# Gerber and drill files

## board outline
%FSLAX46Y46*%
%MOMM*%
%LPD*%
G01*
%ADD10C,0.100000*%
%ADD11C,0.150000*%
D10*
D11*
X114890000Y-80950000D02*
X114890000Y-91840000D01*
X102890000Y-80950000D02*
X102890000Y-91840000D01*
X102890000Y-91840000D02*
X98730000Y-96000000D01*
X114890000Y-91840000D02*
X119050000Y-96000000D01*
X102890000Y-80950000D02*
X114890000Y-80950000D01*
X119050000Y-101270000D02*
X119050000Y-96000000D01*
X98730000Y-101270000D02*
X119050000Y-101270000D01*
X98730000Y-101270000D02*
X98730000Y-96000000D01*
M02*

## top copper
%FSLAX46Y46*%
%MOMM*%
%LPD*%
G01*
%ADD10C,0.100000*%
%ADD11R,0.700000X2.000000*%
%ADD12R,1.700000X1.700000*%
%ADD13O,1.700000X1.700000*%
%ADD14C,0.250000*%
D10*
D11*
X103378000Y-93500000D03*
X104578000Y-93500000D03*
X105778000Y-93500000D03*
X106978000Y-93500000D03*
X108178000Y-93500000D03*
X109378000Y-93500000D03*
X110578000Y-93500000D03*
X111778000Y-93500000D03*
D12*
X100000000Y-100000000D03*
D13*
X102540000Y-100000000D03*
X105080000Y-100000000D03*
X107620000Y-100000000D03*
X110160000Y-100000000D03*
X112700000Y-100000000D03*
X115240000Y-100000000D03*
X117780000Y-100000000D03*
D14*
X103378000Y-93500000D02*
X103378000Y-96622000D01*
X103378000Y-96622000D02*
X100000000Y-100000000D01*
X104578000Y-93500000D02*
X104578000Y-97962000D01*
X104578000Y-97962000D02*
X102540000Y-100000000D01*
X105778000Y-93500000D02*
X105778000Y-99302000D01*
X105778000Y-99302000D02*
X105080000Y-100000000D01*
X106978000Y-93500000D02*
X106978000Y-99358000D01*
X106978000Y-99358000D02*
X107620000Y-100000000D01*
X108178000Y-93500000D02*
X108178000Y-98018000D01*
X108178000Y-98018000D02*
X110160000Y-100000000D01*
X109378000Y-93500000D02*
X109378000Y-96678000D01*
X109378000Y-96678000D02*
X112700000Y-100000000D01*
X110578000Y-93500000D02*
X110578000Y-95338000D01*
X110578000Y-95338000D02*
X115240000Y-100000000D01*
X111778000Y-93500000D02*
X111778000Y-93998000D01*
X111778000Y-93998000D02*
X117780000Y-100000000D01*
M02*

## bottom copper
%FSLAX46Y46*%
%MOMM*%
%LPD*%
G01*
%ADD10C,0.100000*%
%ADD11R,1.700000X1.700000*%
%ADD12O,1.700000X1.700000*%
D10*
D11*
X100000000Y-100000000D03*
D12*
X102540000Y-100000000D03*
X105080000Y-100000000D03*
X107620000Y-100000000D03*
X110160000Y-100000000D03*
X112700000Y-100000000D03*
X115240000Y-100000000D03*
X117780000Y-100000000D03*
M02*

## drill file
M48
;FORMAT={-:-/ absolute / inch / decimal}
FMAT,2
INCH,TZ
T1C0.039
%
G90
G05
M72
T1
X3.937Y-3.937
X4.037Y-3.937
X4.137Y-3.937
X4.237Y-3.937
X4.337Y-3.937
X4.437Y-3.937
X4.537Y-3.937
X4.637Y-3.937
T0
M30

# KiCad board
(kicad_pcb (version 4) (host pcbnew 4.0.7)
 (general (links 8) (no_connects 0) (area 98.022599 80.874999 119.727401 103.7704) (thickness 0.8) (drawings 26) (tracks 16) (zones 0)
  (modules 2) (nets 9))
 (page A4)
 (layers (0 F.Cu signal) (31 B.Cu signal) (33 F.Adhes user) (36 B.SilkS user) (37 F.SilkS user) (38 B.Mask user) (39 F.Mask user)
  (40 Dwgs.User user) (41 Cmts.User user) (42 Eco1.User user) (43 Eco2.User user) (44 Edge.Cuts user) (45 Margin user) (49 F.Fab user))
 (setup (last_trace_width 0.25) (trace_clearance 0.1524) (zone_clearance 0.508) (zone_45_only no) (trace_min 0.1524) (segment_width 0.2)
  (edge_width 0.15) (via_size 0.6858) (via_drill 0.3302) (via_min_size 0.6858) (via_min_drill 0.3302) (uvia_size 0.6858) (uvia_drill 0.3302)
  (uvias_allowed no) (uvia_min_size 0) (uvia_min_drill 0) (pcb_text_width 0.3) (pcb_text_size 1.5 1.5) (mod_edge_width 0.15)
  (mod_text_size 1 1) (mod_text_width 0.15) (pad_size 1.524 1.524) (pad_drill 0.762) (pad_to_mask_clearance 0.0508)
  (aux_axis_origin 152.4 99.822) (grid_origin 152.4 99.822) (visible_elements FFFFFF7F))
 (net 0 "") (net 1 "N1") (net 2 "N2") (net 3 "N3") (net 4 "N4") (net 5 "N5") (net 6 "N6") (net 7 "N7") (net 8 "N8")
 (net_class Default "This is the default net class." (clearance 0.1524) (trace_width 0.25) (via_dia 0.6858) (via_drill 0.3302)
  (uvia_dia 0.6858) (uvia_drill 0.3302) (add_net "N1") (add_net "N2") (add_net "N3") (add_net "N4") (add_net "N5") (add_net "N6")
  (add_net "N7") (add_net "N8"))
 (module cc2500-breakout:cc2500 (layer F.Cu) (at 103.378 93.5)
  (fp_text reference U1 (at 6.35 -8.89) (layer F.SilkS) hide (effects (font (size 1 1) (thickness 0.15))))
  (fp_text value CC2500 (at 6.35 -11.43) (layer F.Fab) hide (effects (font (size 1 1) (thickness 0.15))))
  (pad 1 smd rect (at 0 0) (size 0.7 2) (layers F.Cu F.Mask) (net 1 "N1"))
  (pad 2 smd rect (at 1.2 0) (size 0.7 2) (layers F.Cu F.Mask) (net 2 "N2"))
  (pad 3 smd rect (at 2.4 0) (size 0.7 2) (layers F.Cu F.Mask) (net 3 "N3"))
  (pad 4 smd rect (at 3.6 0) (size 0.7 2) (layers F.Cu F.Mask) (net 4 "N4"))
  (pad 5 smd rect (at 4.8 0) (size 0.7 2) (layers F.Cu F.Mask) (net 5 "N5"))
  (pad 6 smd rect (at 6 0) (size 0.7 2) (layers F.Cu F.Mask) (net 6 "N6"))
  (pad 7 smd rect (at 7.2 0) (size 0.7 2) (layers F.Cu F.Mask) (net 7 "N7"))
  (pad 8 smd rect (at 8.4 0) (size 0.7 2) (layers F.Cu F.Mask) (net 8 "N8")))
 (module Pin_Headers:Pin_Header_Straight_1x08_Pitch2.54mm (layer F.Cu) (at 100 100 90)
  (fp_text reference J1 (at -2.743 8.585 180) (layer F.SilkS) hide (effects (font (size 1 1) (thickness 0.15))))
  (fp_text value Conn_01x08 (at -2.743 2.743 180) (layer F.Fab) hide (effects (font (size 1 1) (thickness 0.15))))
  (pad 1 thru_hole rect (at 0 0 90) (size 1.7 1.7) (drill 1) (layers *.Cu *.Mask) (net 1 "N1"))
  (pad 2 thru_hole oval (at 0 2.54 90) (size 1.7 1.7) (drill 1) (layers *.Cu *.Mask) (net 2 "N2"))
  (pad 3 thru_hole oval (at 0 5.08 90) (size 1.7 1.7) (drill 1) (layers *.Cu *.Mask) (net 3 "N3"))
  (pad 4 thru_hole oval (at 0 7.62 90) (size 1.7 1.7) (drill 1) (layers *.Cu *.Mask) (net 4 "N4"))
  (pad 5 thru_hole oval (at 0 10.16 90) (size 1.7 1.7) (drill 1) (layers *.Cu *.Mask) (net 5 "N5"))
  (pad 6 thru_hole oval (at 0 12.7 90) (size 1.7 1.7) (drill 1) (layers *.Cu *.Mask) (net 6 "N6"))
  (pad 7 thru_hole oval (at 0 15.24 90) (size 1.7 1.7) (drill 1) (layers *.Cu *.Mask) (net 7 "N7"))
  (pad 8 thru_hole oval (at 0 17.78 90) (size 1.7 1.7) (drill 1) (layers *.Cu *.Mask) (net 8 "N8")))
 (gr_line (start 114.89 80.95) (end 114.89 91.84) (angle 90) (layer Edge.Cuts) (width 0.15))
 (gr_line (start 102.89 80.95) (end 102.89 91.84) (angle 90) (layer Edge.Cuts) (width 0.15))
 (gr_line (start 102.89 91.84) (end 98.73 96) (angle 90) (layer Edge.Cuts) (width 0.15))
 (gr_line (start 114.89 91.84) (end 119.05 96) (angle 90) (layer Edge.Cuts) (width 0.15))
 (gr_line (start 102.89 80.95) (end 114.89 80.95) (angle 90) (layer Edge.Cuts) (width 0.15))
 (gr_line (start 119.05 101.27) (end 119.05 96) (angle 90) (layer Edge.Cuts) (width 0.15))
 (gr_line (start 98.73 101.27) (end 119.05 101.27) (angle 90) (layer Edge.Cuts) (width 0.15))
 (gr_line (start 98.73 101.27) (end 98.73 96) (angle 90) (layer Edge.Cuts) (width 0.15))
 (segment (start 103.378 93.5) (end 103.378 96.622) (width 0.25) (layer F.Cu) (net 1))
 (segment (start 103.378 96.622) (end 100 100) (width 0.25) (layer F.Cu) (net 1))
 (segment (start 104.578 93.5) (end 104.578 97.962) (width 0.25) (layer F.Cu) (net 2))
 (segment (start 104.578 97.962) (end 102.54 100) (width 0.25) (layer F.Cu) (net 2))
 (segment (start 105.778 93.5) (end 105.778 99.302) (width 0.25) (layer F.Cu) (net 3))
 (segment (start 105.778 99.302) (end 105.08 100) (width 0.25) (layer F.Cu) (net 3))
 (segment (start 106.978 93.5) (end 106.978 99.358) (width 0.25) (layer F.Cu) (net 4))
 (segment (start 106.978 99.358) (end 107.62 100) (width 0.25) (layer F.Cu) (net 4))
 (segment (start 108.178 93.5) (end 108.178 98.018) (width 0.25) (layer F.Cu) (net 5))
 (segment (start 108.178 98.018) (end 110.16 100) (width 0.25) (layer F.Cu) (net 5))
 (segment (start 109.378 93.5) (end 109.378 96.678) (width 0.25) (layer F.Cu) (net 6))
 (segment (start 109.378 96.678) (end 112.7 100) (width 0.25) (layer F.Cu) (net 6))
 (segment (start 110.578 93.5) (end 110.578 95.338) (width 0.25) (layer F.Cu) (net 7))
 (segment (start 110.578 95.338) (end 115.24 100) (width 0.25) (layer F.Cu) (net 7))
 (segment (start 111.778 93.5) (end 111.778 93.998) (width 0.25) (layer F.Cu) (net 8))
 (segment (start 111.778 93.998) (end 117.78 100) (width 0.25) (layer F.Cu) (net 8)))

